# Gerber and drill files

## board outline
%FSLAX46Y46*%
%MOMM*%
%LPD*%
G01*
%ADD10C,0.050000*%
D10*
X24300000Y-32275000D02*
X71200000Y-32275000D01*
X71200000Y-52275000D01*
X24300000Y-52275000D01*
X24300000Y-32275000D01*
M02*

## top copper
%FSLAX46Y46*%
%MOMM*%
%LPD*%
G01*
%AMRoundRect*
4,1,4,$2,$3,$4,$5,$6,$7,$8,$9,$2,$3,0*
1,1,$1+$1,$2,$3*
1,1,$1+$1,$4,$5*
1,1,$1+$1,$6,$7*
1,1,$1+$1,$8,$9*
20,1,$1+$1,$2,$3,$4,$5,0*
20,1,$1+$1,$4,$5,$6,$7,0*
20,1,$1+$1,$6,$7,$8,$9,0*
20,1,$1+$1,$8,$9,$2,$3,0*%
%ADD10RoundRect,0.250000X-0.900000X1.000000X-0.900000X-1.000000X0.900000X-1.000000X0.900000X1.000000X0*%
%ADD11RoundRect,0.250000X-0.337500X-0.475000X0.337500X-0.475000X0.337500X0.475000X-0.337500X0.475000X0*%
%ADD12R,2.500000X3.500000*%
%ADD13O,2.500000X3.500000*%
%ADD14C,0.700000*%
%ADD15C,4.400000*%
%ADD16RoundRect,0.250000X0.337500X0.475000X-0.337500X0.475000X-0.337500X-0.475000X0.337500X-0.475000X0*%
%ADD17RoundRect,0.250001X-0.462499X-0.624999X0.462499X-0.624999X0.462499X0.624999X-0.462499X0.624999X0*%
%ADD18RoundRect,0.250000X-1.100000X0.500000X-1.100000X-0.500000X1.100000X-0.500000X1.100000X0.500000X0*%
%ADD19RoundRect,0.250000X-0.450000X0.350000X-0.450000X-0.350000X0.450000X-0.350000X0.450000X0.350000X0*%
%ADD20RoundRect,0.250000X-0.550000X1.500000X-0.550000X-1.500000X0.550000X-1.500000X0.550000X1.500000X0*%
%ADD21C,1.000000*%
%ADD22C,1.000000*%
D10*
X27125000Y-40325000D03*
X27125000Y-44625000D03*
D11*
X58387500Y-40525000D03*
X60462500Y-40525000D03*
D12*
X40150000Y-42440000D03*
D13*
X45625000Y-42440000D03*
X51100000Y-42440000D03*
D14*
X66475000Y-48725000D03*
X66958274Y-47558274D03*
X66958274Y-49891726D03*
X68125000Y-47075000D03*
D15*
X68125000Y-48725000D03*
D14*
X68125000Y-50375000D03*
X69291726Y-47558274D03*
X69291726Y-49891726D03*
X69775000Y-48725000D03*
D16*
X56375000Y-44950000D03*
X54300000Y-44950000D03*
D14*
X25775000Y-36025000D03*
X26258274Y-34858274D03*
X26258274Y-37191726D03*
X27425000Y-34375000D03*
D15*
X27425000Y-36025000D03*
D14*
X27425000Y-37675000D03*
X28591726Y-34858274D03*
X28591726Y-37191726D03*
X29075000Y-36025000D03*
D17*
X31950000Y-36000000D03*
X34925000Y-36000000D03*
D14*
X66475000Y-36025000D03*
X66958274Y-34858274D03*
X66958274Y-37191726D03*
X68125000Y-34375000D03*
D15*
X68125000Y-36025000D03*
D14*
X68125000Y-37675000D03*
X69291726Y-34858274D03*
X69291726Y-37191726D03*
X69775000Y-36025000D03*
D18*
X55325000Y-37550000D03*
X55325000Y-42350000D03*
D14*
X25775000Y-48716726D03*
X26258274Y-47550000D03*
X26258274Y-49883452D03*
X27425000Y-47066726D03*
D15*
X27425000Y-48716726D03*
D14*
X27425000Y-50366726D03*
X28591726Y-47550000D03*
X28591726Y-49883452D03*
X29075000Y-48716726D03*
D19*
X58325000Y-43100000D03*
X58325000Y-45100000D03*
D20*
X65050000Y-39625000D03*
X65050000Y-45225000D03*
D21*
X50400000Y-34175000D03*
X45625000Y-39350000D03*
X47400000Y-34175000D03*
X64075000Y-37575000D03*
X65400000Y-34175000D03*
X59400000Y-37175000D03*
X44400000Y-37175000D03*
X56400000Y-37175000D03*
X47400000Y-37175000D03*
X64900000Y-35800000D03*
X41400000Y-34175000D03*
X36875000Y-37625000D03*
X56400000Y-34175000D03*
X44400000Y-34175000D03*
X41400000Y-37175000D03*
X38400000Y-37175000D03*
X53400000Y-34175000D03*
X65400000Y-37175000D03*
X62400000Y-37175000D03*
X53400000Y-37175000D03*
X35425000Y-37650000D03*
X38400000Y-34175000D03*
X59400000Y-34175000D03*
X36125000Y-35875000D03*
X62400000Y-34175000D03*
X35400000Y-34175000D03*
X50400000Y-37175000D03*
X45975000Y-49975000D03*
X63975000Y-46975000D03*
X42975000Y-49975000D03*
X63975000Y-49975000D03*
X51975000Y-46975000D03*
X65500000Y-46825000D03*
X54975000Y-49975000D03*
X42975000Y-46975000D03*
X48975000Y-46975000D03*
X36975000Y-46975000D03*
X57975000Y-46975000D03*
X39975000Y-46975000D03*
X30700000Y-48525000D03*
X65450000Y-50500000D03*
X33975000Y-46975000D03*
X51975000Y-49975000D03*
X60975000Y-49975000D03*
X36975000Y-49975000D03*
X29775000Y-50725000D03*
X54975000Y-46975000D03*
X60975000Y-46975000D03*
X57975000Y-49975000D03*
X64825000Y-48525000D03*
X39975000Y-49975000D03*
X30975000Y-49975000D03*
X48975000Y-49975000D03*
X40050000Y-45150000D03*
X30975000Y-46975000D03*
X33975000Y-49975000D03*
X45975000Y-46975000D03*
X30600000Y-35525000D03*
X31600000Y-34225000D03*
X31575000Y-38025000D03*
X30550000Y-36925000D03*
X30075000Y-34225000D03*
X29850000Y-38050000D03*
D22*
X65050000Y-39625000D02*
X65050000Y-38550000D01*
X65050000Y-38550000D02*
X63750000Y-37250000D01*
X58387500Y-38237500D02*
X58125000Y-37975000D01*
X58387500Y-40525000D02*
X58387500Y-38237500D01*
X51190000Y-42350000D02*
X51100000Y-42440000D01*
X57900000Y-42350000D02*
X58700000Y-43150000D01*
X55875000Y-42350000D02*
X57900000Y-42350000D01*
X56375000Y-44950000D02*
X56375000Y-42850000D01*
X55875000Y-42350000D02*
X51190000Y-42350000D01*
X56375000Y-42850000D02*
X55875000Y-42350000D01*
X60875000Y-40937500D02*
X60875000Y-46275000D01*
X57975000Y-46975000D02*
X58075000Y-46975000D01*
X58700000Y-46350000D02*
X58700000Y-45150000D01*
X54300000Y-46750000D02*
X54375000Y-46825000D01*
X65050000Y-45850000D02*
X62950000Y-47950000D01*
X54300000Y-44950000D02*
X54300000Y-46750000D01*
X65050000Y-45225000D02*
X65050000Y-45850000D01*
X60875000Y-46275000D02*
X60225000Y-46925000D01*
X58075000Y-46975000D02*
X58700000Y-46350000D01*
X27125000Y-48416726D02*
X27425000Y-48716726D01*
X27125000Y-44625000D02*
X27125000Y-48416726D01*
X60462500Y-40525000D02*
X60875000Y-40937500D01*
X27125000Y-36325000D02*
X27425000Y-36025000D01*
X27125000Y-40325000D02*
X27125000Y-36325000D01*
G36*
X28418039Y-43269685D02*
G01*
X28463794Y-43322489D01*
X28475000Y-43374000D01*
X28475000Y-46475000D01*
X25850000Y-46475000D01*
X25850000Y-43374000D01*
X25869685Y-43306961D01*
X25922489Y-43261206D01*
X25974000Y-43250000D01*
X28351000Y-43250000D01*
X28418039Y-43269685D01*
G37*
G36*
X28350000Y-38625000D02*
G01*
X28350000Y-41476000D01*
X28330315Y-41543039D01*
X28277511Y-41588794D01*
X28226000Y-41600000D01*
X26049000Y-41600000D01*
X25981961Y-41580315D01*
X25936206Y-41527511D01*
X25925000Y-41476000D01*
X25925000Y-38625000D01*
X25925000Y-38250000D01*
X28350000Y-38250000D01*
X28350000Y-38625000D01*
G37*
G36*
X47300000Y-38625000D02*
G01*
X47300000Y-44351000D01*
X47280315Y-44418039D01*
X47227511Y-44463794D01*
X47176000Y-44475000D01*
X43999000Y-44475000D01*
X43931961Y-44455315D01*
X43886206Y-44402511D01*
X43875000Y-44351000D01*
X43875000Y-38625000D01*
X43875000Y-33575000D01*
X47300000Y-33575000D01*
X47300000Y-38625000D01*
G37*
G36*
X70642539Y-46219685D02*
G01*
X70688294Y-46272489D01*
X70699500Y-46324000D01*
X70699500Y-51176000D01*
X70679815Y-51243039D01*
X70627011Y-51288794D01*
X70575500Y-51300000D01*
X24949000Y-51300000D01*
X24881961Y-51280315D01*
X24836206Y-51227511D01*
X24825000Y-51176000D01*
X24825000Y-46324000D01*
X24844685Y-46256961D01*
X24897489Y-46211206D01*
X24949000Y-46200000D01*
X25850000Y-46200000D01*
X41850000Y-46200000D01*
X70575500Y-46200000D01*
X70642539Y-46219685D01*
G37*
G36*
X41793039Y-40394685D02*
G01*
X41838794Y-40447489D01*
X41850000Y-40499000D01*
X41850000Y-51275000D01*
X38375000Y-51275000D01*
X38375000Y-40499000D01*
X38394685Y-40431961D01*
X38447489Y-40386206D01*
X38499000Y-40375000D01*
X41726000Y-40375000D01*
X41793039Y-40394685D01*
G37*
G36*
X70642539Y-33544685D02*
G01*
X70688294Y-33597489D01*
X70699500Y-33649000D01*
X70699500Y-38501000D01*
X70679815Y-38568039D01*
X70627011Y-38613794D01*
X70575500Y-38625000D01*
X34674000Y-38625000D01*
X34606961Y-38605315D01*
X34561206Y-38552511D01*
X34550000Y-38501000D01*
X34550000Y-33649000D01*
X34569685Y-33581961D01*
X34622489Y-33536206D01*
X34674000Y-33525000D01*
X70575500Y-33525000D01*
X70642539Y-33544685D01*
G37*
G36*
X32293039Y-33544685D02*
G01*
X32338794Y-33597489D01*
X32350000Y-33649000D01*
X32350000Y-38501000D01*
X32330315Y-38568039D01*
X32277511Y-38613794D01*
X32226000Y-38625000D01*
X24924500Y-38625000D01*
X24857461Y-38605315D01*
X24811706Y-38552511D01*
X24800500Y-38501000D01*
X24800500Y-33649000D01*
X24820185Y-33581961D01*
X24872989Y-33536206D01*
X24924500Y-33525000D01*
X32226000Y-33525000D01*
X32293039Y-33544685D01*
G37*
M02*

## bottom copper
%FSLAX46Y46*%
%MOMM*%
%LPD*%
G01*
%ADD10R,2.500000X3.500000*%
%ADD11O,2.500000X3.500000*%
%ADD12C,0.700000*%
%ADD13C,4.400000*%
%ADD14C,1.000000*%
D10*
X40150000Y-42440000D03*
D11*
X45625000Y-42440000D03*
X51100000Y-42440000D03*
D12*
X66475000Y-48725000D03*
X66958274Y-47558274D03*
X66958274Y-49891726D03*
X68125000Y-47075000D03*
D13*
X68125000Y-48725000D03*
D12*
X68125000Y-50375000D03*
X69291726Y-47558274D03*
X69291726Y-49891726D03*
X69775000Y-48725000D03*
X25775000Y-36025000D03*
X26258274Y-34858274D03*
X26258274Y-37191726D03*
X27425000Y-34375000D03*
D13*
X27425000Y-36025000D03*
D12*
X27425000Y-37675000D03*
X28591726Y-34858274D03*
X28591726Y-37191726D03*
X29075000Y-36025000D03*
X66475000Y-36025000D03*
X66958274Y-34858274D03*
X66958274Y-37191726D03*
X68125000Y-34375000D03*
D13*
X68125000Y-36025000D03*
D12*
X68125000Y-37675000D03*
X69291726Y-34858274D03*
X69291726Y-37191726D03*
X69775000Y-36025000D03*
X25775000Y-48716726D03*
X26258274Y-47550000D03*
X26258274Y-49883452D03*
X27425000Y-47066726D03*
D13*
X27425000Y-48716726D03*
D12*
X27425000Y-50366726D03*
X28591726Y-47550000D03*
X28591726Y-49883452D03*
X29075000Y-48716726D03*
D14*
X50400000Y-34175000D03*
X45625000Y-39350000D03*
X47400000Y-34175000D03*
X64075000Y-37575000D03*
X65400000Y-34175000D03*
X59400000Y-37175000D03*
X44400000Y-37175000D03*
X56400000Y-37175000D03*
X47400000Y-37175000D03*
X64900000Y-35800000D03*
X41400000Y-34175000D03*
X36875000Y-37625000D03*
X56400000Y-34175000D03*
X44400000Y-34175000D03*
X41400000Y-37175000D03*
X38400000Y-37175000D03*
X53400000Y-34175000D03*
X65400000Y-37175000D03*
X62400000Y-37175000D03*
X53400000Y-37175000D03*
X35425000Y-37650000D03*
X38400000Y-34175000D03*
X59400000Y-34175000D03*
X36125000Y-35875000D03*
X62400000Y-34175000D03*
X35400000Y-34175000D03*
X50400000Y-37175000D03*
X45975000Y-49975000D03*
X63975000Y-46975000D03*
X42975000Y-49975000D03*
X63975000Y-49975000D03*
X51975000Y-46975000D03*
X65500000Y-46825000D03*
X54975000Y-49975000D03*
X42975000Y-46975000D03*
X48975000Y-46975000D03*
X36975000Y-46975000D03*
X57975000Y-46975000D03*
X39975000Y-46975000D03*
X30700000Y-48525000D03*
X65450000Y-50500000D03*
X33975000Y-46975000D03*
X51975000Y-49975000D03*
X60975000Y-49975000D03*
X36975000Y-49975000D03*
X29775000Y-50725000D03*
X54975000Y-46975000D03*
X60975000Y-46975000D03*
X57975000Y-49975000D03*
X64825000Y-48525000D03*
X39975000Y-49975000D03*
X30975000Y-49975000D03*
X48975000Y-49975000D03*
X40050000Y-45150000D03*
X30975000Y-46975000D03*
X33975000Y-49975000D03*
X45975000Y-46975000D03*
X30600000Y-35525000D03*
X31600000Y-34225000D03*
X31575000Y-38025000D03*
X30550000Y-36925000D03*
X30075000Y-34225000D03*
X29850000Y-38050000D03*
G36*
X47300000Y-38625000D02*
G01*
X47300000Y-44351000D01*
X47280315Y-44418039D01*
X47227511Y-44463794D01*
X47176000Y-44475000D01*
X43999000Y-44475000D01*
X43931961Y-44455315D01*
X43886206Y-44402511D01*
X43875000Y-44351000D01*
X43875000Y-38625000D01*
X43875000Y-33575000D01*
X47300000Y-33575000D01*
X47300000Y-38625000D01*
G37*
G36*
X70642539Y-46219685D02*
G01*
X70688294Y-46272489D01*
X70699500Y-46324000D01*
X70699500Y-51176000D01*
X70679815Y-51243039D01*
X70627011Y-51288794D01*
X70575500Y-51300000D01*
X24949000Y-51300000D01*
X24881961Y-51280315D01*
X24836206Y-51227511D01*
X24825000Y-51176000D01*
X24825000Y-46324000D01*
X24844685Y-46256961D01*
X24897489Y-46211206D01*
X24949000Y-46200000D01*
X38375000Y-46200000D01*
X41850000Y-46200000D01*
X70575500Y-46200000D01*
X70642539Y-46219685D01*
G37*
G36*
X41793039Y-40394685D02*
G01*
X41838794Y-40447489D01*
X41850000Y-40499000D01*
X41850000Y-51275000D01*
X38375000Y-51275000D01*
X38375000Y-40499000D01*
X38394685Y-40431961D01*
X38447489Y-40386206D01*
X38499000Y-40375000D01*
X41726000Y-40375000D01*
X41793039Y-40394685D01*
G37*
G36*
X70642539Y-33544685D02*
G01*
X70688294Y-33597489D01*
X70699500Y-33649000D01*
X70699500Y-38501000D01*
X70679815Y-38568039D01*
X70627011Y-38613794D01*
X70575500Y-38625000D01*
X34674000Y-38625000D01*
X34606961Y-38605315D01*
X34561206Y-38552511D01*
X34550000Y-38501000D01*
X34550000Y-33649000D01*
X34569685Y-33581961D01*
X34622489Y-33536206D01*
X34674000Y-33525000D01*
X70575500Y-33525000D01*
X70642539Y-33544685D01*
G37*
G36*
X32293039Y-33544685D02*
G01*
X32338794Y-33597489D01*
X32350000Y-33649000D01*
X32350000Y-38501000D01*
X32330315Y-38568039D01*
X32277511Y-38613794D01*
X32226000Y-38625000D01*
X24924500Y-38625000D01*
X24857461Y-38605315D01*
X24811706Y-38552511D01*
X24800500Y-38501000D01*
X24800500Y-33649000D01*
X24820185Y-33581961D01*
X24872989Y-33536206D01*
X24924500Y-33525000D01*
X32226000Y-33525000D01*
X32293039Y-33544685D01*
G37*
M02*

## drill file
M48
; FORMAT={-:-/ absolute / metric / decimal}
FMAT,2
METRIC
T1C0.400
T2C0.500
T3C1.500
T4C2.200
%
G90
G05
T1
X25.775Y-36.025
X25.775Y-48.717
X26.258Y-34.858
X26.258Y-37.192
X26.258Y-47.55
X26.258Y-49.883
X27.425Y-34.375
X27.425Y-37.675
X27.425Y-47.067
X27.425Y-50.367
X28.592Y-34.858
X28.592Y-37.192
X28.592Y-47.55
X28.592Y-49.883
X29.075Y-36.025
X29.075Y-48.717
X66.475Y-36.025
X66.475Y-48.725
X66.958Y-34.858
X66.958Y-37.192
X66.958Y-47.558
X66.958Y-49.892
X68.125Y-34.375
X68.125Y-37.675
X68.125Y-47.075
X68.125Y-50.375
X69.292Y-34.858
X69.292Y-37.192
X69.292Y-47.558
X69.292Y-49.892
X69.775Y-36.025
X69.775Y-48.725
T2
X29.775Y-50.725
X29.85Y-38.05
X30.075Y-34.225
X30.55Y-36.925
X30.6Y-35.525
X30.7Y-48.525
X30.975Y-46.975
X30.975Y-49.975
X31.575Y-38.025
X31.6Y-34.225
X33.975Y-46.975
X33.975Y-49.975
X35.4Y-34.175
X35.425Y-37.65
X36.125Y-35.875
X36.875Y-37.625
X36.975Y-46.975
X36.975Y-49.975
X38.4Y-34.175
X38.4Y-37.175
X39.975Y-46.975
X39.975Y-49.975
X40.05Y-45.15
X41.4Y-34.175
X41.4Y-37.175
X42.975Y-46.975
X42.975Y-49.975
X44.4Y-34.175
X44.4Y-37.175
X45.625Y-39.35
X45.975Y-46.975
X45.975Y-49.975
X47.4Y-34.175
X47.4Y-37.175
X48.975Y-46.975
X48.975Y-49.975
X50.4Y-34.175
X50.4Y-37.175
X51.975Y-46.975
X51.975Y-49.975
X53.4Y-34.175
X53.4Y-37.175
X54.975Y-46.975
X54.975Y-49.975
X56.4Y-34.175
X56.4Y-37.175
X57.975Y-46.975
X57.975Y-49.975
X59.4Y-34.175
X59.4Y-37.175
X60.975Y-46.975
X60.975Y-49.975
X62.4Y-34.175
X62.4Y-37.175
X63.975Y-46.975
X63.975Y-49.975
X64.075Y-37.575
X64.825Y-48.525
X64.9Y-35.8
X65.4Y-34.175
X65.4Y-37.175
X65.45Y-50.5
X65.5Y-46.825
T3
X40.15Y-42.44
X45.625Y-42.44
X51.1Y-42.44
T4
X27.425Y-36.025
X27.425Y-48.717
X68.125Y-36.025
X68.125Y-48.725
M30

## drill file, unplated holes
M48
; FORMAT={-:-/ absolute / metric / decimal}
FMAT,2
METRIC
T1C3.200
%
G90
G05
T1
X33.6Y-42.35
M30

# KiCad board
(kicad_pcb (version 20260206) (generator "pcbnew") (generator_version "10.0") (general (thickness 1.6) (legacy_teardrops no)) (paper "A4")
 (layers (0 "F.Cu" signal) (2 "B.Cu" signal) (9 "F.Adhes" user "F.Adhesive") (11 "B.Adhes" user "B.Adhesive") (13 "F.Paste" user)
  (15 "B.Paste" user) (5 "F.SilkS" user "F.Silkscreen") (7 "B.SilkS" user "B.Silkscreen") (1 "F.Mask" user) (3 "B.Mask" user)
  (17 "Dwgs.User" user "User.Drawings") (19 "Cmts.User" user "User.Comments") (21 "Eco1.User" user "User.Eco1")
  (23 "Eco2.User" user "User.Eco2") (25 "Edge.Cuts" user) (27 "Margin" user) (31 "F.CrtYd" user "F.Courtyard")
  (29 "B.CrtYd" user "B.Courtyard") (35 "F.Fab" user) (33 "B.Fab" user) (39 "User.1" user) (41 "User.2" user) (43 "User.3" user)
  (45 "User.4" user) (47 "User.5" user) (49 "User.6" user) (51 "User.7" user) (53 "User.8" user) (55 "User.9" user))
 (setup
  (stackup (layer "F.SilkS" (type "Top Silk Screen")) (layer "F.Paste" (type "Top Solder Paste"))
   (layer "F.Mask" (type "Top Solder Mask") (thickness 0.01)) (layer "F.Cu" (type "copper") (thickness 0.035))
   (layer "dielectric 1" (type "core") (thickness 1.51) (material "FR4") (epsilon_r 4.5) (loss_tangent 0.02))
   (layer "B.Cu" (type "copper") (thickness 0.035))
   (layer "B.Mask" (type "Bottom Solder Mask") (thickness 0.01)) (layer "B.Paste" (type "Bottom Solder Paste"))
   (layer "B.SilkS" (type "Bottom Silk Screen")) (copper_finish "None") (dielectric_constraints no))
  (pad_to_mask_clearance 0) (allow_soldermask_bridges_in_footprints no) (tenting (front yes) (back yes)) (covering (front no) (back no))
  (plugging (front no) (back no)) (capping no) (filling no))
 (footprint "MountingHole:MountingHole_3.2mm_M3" (layer "F.Cu") (at 33.6 42.35)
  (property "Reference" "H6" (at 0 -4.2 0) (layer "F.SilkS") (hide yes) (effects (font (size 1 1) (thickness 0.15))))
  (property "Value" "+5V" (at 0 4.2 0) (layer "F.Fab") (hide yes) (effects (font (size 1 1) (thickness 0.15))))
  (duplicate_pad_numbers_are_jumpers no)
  (pad "" np_thru_hole circle (at 0 0) (size 3.2 3.2) (drill 3.2) (layers "*.Cu" "*.Mask")))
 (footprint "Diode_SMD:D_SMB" (layer "F.Cu") (at 27.125 42.475 -90)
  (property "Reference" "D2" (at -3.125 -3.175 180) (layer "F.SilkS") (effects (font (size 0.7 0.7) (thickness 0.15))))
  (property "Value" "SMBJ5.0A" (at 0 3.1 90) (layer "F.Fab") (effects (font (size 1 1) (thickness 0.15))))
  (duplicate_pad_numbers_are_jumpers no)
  (pad "1" smd roundrect (at -2.15 0 270) (size 2.5 2.3) (layers "F.Cu" "F.Mask" "F.Paste") (roundrect_rratio 0.1086956522) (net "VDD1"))
  (pad "2" smd roundrect (at 2.15 0 270) (size 2.5 2.3) (layers "F.Cu" "F.Mask" "F.Paste") (roundrect_rratio 0.1086956522) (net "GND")))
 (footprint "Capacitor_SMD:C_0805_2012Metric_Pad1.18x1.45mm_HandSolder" (layer "F.Cu") (at 59.425 40.525)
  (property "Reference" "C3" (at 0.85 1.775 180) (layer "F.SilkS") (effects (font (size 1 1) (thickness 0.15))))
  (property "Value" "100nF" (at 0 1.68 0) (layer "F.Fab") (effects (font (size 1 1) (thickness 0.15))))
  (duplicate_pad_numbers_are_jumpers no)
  (pad "1" smd roundrect (at -1.0375 0) (size 1.175 1.45) (layers "F.Cu" "F.Mask" "F.Paste") (roundrect_rratio 0.212766) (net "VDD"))
  (pad "2" smd roundrect (at 1.0375 0) (size 1.175 1.45) (layers "F.Cu" "F.Mask" "F.Paste") (roundrect_rratio 0.212766) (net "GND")))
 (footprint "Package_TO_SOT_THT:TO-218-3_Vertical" (layer "F.Cu") (at 40.15 42.44)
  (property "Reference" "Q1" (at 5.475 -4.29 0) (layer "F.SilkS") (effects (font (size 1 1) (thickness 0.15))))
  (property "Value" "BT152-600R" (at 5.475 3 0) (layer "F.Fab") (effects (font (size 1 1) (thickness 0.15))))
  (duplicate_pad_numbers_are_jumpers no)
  (pad "1" thru_hole rect (at 0 0) (size 2.5 3.5) (drill 1.5) (layers "*.Cu" "*.Mask") (remove_unused_layers no) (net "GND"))
  (pad "2" thru_hole oval (at 5.475 0) (size 2.5 3.5) (drill 1.5) (layers "*.Cu" "*.Mask") (remove_unused_layers no) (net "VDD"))
  (pad "3" thru_hole oval (at 10.95 0) (size 2.5 3.5) (drill 1.5) (layers "*.Cu" "*.Mask") (remove_unused_layers no) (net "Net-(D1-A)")))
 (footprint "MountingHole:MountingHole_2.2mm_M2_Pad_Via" (layer "F.Cu") (at 68.125 48.725)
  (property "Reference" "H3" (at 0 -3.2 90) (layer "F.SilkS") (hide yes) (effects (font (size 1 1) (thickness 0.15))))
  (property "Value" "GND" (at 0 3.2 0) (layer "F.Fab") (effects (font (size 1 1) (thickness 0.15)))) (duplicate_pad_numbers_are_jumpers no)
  (pad "1" thru_hole circle (at -1.65 0) (size 0.7 0.7) (drill 0.4) (layers "*.Cu" "*.Mask") (remove_unused_layers no) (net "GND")
   (zone_connect 2))
  (pad "1" thru_hole circle (at -1.166726 -1.166726) (size 0.7 0.7) (drill 0.4) (layers "*.Cu" "*.Mask") (remove_unused_layers no)
   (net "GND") (zone_connect 2))
  (pad "1" thru_hole circle (at -1.166726 1.166726) (size 0.7 0.7) (drill 0.4) (layers "*.Cu" "*.Mask") (remove_unused_layers no)
   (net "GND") (zone_connect 2))
  (pad "1" thru_hole circle (at 0 -1.65) (size 0.7 0.7) (drill 0.4) (layers "*.Cu" "*.Mask") (remove_unused_layers no) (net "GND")
   (zone_connect 2))
  (pad "1" thru_hole circle (at 0 0) (size 4.4 4.4) (drill 2.2) (layers "*.Cu" "*.Mask") (remove_unused_layers no) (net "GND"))
  (pad "1" thru_hole circle (at 0 1.65) (size 0.7 0.7) (drill 0.4) (layers "*.Cu" "*.Mask") (remove_unused_layers no) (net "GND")
   (zone_connect 2))
  (pad "1" thru_hole circle (at 1.166726 -1.166726) (size 0.7 0.7) (drill 0.4) (layers "*.Cu" "*.Mask") (remove_unused_layers no)
   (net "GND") (zone_connect 2))
  (pad "1" thru_hole circle (at 1.166726 1.166726) (size 0.7 0.7) (drill 0.4) (layers "*.Cu" "*.Mask") (remove_unused_layers no) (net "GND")
   (zone_connect 2))
  (pad "1" thru_hole circle (at 1.65 0) (size 0.7 0.7) (drill 0.4) (layers "*.Cu" "*.Mask") (remove_unused_layers no) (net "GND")
   (zone_connect 2)))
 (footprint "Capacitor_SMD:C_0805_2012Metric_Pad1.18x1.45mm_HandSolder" (layer "F.Cu") (at 55.3375 44.95 180)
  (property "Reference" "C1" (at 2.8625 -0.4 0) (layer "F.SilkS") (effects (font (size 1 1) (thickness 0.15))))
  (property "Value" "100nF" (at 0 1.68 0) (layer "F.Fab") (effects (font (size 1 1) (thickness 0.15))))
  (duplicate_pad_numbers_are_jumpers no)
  (pad "1" smd roundrect (at -1.0375 0 180) (size 1.175 1.45) (layers "F.Cu" "F.Mask" "F.Paste") (roundrect_rratio 0.212766)
   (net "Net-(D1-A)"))
  (pad "2" smd roundrect (at 1.0375 0 180) (size 1.175 1.45) (layers "F.Cu" "F.Mask" "F.Paste") (roundrect_rratio 0.212766) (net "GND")))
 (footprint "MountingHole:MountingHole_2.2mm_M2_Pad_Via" (layer "F.Cu") (at 27.425 36.025)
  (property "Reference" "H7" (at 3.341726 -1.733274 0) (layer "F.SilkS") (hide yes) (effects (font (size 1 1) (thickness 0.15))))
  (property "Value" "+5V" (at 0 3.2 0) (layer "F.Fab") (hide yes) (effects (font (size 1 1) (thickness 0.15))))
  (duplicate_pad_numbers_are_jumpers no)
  (pad "1" thru_hole circle (at -1.65 0) (size 0.7 0.7) (drill 0.4) (layers "*.Cu" "*.Mask") (remove_unused_layers no) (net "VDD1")
   (zone_connect 2))
  (pad "1" thru_hole circle (at -1.166726 -1.166726) (size 0.7 0.7) (drill 0.4) (layers "*.Cu" "*.Mask") (remove_unused_layers no)
   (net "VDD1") (zone_connect 2))
  (pad "1" thru_hole circle (at -1.166726 1.166726) (size 0.7 0.7) (drill 0.4) (layers "*.Cu" "*.Mask") (remove_unused_layers no)
   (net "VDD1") (zone_connect 2))
  (pad "1" thru_hole circle (at 0 -1.65) (size 0.7 0.7) (drill 0.4) (layers "*.Cu" "*.Mask") (remove_unused_layers no) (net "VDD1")
   (zone_connect 2))
  (pad "1" thru_hole circle (at 0 0) (size 4.4 4.4) (drill 2.2) (layers "*.Cu" "*.Mask") (remove_unused_layers no) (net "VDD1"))
  (pad "1" thru_hole circle (at 0 1.65) (size 0.7 0.7) (drill 0.4) (layers "*.Cu" "*.Mask") (remove_unused_layers no) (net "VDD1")
   (zone_connect 2))
  (pad "1" thru_hole circle (at 1.166726 -1.166726) (size 0.7 0.7) (drill 0.4) (layers "*.Cu" "*.Mask") (remove_unused_layers no)
   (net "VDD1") (zone_connect 2))
  (pad "1" thru_hole circle (at 1.166726 1.166726) (size 0.7 0.7) (drill 0.4) (layers "*.Cu" "*.Mask") (remove_unused_layers no)
   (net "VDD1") (zone_connect 2))
  (pad "1" thru_hole circle (at 1.65 0) (size 0.7 0.7) (drill 0.4) (layers "*.Cu" "*.Mask") (remove_unused_layers no) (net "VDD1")
   (zone_connect 2)))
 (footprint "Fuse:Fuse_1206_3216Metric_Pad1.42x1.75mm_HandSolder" (layer "F.Cu") (at 33.4375 36)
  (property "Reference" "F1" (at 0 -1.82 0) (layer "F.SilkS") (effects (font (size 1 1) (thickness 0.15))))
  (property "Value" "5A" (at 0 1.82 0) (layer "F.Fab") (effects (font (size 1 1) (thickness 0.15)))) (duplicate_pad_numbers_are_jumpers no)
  (pad "1" smd roundrect (at -1.4875 0) (size 1.425 1.75) (layers "F.Cu" "F.Mask" "F.Paste") (roundrect_rratio 0.175439) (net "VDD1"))
  (pad "2" smd roundrect (at 1.4875 0) (size 1.425 1.75) (layers "F.Cu" "F.Mask" "F.Paste") (roundrect_rratio 0.175439) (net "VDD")))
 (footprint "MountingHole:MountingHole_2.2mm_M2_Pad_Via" (layer "F.Cu") (at 68.125 36.025)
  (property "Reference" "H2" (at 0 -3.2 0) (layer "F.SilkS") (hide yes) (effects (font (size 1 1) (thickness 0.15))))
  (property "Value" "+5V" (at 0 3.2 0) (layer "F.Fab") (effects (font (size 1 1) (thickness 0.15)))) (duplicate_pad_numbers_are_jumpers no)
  (pad "1" thru_hole circle (at -1.65 0) (size 0.7 0.7) (drill 0.4) (layers "*.Cu" "*.Mask") (remove_unused_layers no) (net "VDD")
   (zone_connect 2))
  (pad "1" thru_hole circle (at -1.166726 -1.166726) (size 0.7 0.7) (drill 0.4) (layers "*.Cu" "*.Mask") (remove_unused_layers no)
   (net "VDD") (zone_connect 2))
  (pad "1" thru_hole circle (at -1.166726 1.166726) (size 0.7 0.7) (drill 0.4) (layers "*.Cu" "*.Mask") (remove_unused_layers no)
   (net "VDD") (zone_connect 2))
  (pad "1" thru_hole circle (at 0 -1.65) (size 0.7 0.7) (drill 0.4) (layers "*.Cu" "*.Mask") (remove_unused_layers no) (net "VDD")
   (zone_connect 2))
  (pad "1" thru_hole circle (at 0 0) (size 4.4 4.4) (drill 2.2) (layers "*.Cu" "*.Mask") (remove_unused_layers no) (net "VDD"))
  (pad "1" thru_hole circle (at 0 1.65) (size 0.7 0.7) (drill 0.4) (layers "*.Cu" "*.Mask") (remove_unused_layers no) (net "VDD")
   (zone_connect 2))
  (pad "1" thru_hole circle (at 1.166726 -1.166726) (size 0.7 0.7) (drill 0.4) (layers "*.Cu" "*.Mask") (remove_unused_layers no)
   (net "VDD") (zone_connect 2))
  (pad "1" thru_hole circle (at 1.166726 1.166726) (size 0.7 0.7) (drill 0.4) (layers "*.Cu" "*.Mask") (remove_unused_layers no) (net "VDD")
   (zone_connect 2))
  (pad "1" thru_hole circle (at 1.65 0) (size 0.7 0.7) (drill 0.4) (layers "*.Cu" "*.Mask") (remove_unused_layers no) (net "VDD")
   (zone_connect 2)))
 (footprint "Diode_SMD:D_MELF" (layer "F.Cu") (at 55.325 39.95 -90)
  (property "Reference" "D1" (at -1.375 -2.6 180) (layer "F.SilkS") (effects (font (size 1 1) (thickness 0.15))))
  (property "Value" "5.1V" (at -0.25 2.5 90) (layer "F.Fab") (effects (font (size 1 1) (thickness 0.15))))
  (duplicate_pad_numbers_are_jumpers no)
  (pad "1" smd roundrect (at -2.4 0 270) (size 1.5 2.7) (layers "F.Cu" "F.Mask" "F.Paste") (roundrect_rratio 0.1666666667) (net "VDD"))
  (pad "2" smd roundrect (at 2.4 0 270) (size 1.5 2.7) (layers "F.Cu" "F.Mask" "F.Paste") (roundrect_rratio 0.1666666667) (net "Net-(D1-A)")))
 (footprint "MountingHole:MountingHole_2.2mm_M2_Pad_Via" (layer "F.Cu") (at 27.425 48.716726)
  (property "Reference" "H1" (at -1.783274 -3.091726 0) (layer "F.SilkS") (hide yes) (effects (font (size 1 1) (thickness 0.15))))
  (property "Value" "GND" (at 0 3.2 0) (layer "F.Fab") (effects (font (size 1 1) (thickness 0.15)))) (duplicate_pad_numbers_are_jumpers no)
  (pad "1" thru_hole circle (at -1.65 0) (size 0.7 0.7) (drill 0.4) (layers "*.Cu" "*.Mask") (remove_unused_layers no) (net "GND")
   (zone_connect 2))
  (pad "1" thru_hole circle (at -1.166726 -1.166726) (size 0.7 0.7) (drill 0.4) (layers "*.Cu" "*.Mask") (remove_unused_layers no)
   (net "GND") (zone_connect 2))
  (pad "1" thru_hole circle (at -1.166726 1.166726) (size 0.7 0.7) (drill 0.4) (layers "*.Cu" "*.Mask") (remove_unused_layers no)
   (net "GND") (zone_connect 2))
  (pad "1" thru_hole circle (at 0 -1.65) (size 0.7 0.7) (drill 0.4) (layers "*.Cu" "*.Mask") (remove_unused_layers no) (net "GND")
   (zone_connect 2))
  (pad "1" thru_hole circle (at 0 0) (size 4.4 4.4) (drill 2.2) (layers "*.Cu" "*.Mask") (remove_unused_layers no) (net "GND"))
  (pad "1" thru_hole circle (at 0 1.65) (size 0.7 0.7) (drill 0.4) (layers "*.Cu" "*.Mask") (remove_unused_layers no) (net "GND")
   (zone_connect 2))
  (pad "1" thru_hole circle (at 1.166726 -1.166726) (size 0.7 0.7) (drill 0.4) (layers "*.Cu" "*.Mask") (remove_unused_layers no)
   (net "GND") (zone_connect 2))
  (pad "1" thru_hole circle (at 1.166726 1.166726) (size 0.7 0.7) (drill 0.4) (layers "*.Cu" "*.Mask") (remove_unused_layers no) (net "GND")
   (zone_connect 2))
  (pad "1" thru_hole circle (at 1.65 0) (size 0.7 0.7) (drill 0.4) (layers "*.Cu" "*.Mask") (remove_unused_layers no) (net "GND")
   (zone_connect 2)))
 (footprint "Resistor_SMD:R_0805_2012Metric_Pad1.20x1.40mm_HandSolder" (layer "F.Cu") (at 58.325 44.1 -90)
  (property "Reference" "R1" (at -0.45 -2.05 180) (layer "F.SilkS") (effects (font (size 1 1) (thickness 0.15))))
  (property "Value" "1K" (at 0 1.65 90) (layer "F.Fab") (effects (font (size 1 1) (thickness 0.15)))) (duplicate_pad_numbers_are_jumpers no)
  (pad "1" smd roundrect (at -1 0 270) (size 1.2 1.4) (layers "F.Cu" "F.Mask" "F.Paste") (roundrect_rratio 0.208333) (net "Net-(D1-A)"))
  (pad "2" smd roundrect (at 1 0 270) (size 1.2 1.4) (layers "F.Cu" "F.Mask" "F.Paste") (roundrect_rratio 0.208333) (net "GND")))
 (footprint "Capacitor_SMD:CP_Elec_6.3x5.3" (layer "F.Cu") (at 65.05 42.425 -90)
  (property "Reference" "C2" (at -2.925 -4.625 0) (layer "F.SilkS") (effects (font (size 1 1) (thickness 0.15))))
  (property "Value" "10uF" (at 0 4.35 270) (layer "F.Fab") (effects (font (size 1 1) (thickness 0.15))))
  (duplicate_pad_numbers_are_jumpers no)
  (pad "1" smd roundrect (at -2.8 0 270) (size 3.5 1.6) (layers "F.Cu" "F.Mask" "F.Paste") (roundrect_rratio 0.15625) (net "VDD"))
  (pad "2" smd roundrect (at 2.8 0 270) (size 3.5 1.6) (layers "F.Cu" "F.Mask" "F.Paste") (roundrect_rratio 0.15625) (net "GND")))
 (gr_rect (start 24.3 32.275) (end 71.2 52.275) (stroke (width 0.05) (type default)) (fill no) (layer "Edge.Cuts"))
 (segment (start 27.125 36.325) (end 27.425 36.025) (width 1) (layer "F.Cu") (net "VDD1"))
 (segment (start 27.125 40.325) (end 27.125 36.325) (width 1) (layer "F.Cu") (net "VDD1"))
 (via (at 30.6 35.525) (size 1) (drill 0.5) (layers "F.Cu" "B.Cu") (free yes) (capping no) (covering (front no) (back no))
  (plugging (front no) (back no)) (filling no) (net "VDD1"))
 (via (at 31.6 34.225) (size 1) (drill 0.5) (layers "F.Cu" "B.Cu") (free yes) (capping no) (covering (front no) (back no))
  (plugging (front no) (back no)) (filling no) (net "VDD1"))
 (via (at 31.575 38.025) (size 1) (drill 0.5) (layers "F.Cu" "B.Cu") (free yes) (capping no) (covering (front no) (back no))
  (plugging (front no) (back no)) (filling no) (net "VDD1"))
 (via (at 30.55 36.925) (size 1) (drill 0.5) (layers "F.Cu" "B.Cu") (free yes) (capping no) (covering (front no) (back no))
  (plugging (front no) (back no)) (filling no) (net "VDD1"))
 (via (at 30.075 34.225) (size 1) (drill 0.5) (layers "F.Cu" "B.Cu") (free yes) (capping no) (covering (front no) (back no))
  (plugging (front no) (back no)) (filling no) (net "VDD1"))
 (via (at 29.85 38.05) (size 1) (drill 0.5) (layers "F.Cu" "B.Cu") (free yes) (capping no) (covering (front no) (back no))
  (plugging (front no) (back no)) (filling no) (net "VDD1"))
 (segment (start 60.875 40.9375) (end 60.875 46.275) (width 1) (layer "F.Cu") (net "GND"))
 (segment (start 57.975 46.975) (end 58.075 46.975) (width 1) (layer "F.Cu") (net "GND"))
 (segment (start 58.7 46.35) (end 58.7 45.15) (width 1) (layer "F.Cu") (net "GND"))
 (segment (start 54.3 46.75) (end 54.375 46.825) (width 1) (layer "F.Cu") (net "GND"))
 (segment (start 65.05 45.85) (end 62.95 47.95) (width 1) (layer "F.Cu") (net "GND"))
 (segment (start 54.3 44.95) (end 54.3 46.75) (width 1) (layer "F.Cu") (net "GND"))
 (segment (start 65.05 45.225) (end 65.05 45.85) (width 1) (layer "F.Cu") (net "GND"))
 (segment (start 60.875 46.275) (end 60.225 46.925) (width 1) (layer "F.Cu") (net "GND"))
 (segment (start 58.075 46.975) (end 58.7 46.35) (width 1) (layer "F.Cu") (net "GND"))
 (segment (start 27.125 48.416726) (end 27.425 48.716726) (width 1) (layer "F.Cu") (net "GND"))
 (segment (start 27.125 44.625) (end 27.125 48.416726) (width 1) (layer "F.Cu") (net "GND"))
 (segment (start 60.4625 40.525) (end 60.875 40.9375) (width 1) (layer "F.Cu") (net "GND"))
 (via (at 45.975 49.975) (size 1) (drill 0.5) (layers "F.Cu" "B.Cu") (free yes) (capping no) (covering (front no) (back no))
  (plugging (front no) (back no)) (filling no) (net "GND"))
 (via (at 63.975 46.975) (size 1) (drill 0.5) (layers "F.Cu" "B.Cu") (free yes) (capping no) (covering (front no) (back no))
  (plugging (front no) (back no)) (filling no) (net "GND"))
 (via (at 42.975 49.975) (size 1) (drill 0.5) (layers "F.Cu" "B.Cu") (free yes) (capping no) (covering (front no) (back no))
  (plugging (front no) (back no)) (filling no) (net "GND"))
 (via (at 63.975 49.975) (size 1) (drill 0.5) (layers "F.Cu" "B.Cu") (free yes) (capping no) (covering (front no) (back no))
  (plugging (front no) (back no)) (filling no) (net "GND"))
 (via (at 51.975 46.975) (size 1) (drill 0.5) (layers "F.Cu" "B.Cu") (free yes) (capping no) (covering (front no) (back no))
  (plugging (front no) (back no)) (filling no) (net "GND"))
 (via (at 65.5 46.825) (size 1) (drill 0.5) (layers "F.Cu" "B.Cu") (free yes) (capping no) (covering (front no) (back no))
  (plugging (front no) (back no)) (filling no) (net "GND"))
 (via (at 54.975 49.975) (size 1) (drill 0.5) (layers "F.Cu" "B.Cu") (free yes) (capping no) (covering (front no) (back no))
  (plugging (front no) (back no)) (filling no) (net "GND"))
 (via (at 42.975 46.975) (size 1) (drill 0.5) (layers "F.Cu" "B.Cu") (free yes) (capping no) (covering (front no) (back no))
  (plugging (front no) (back no)) (filling no) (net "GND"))
 (via (at 48.975 46.975) (size 1) (drill 0.5) (layers "F.Cu" "B.Cu") (free yes) (capping no) (covering (front no) (back no))
  (plugging (front no) (back no)) (filling no) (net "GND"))
 (via (at 36.975 46.975) (size 1) (drill 0.5) (layers "F.Cu" "B.Cu") (free yes) (capping no) (covering (front no) (back no))
  (plugging (front no) (back no)) (filling no) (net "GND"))
 (via (at 57.975 46.975) (size 1) (drill 0.5) (layers "F.Cu" "B.Cu") (free yes) (capping no) (covering (front no) (back no))
  (plugging (front no) (back no)) (filling no) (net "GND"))
 (via (at 39.975 46.975) (size 1) (drill 0.5) (layers "F.Cu" "B.Cu") (free yes) (capping no) (covering (front no) (back no))
  (plugging (front no) (back no)) (filling no) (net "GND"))
 (via (at 30.7 48.525) (size 1) (drill 0.5) (layers "F.Cu" "B.Cu") (free yes) (capping no) (covering (front no) (back no))
  (plugging (front no) (back no)) (filling no) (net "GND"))
 (via (at 65.45 50.5) (size 1) (drill 0.5) (layers "F.Cu" "B.Cu") (free yes) (capping no) (covering (front no) (back no))
  (plugging (front no) (back no)) (filling no) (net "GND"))
 (via (at 33.975 46.975) (size 1) (drill 0.5) (layers "F.Cu" "B.Cu") (free yes) (capping no) (covering (front no) (back no))
  (plugging (front no) (back no)) (filling no) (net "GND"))
 (via (at 51.975 49.975) (size 1) (drill 0.5) (layers "F.Cu" "B.Cu") (free yes) (capping no) (covering (front no) (back no))
  (plugging (front no) (back no)) (filling no) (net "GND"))
 (via (at 60.975 49.975) (size 1) (drill 0.5) (layers "F.Cu" "B.Cu") (free yes) (capping no) (covering (front no) (back no))
  (plugging (front no) (back no)) (filling no) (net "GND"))
 (via (at 36.975 49.975) (size 1) (drill 0.5) (layers "F.Cu" "B.Cu") (free yes) (capping no) (covering (front no) (back no))
  (plugging (front no) (back no)) (filling no) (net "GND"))
 (via (at 29.775 50.725) (size 1) (drill 0.5) (layers "F.Cu" "B.Cu") (free yes) (capping no) (covering (front no) (back no))
  (plugging (front no) (back no)) (filling no) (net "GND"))
 (via (at 54.975 46.975) (size 1) (drill 0.5) (layers "F.Cu" "B.Cu") (free yes) (capping no) (covering (front no) (back no))
  (plugging (front no) (back no)) (filling no) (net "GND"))
 (via (at 60.975 46.975) (size 1) (drill 0.5) (layers "F.Cu" "B.Cu") (free yes) (capping no) (covering (front no) (back no))
  (plugging (front no) (back no)) (filling no) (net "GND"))
 (via (at 57.975 49.975) (size 1) (drill 0.5) (layers "F.Cu" "B.Cu") (free yes) (capping no) (covering (front no) (back no))
  (plugging (front no) (back no)) (filling no) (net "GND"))
 (via (at 64.825 48.525) (size 1) (drill 0.5) (layers "F.Cu" "B.Cu") (free yes) (capping no) (covering (front no) (back no))
  (plugging (front no) (back no)) (filling no) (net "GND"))
 (via (at 39.975 49.975) (size 1) (drill 0.5) (layers "F.Cu" "B.Cu") (free yes) (capping no) (covering (front no) (back no))
  (plugging (front no) (back no)) (filling no) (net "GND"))
 (via (at 30.975 49.975) (size 1) (drill 0.5) (layers "F.Cu" "B.Cu") (free yes) (capping no) (covering (front no) (back no))
  (plugging (front no) (back no)) (filling no) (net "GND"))
 (via (at 48.975 49.975) (size 1) (drill 0.5) (layers "F.Cu" "B.Cu") (free yes) (capping no) (covering (front no) (back no))
  (plugging (front no) (back no)) (filling no) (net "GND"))
 (via (at 40.05 45.15) (size 1) (drill 0.5) (layers "F.Cu" "B.Cu") (free yes) (capping no) (covering (front no) (back no))
  (plugging (front no) (back no)) (filling no) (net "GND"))
 (via (at 30.975 46.975) (size 1) (drill 0.5) (layers "F.Cu" "B.Cu") (free yes) (capping no) (covering (front no) (back no))
  (plugging (front no) (back no)) (filling no) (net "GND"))
 (via (at 33.975 49.975) (size 1) (drill 0.5) (layers "F.Cu" "B.Cu") (free yes) (capping no) (covering (front no) (back no))
  (plugging (front no) (back no)) (filling no) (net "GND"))
 (via (at 45.975 46.975) (size 1) (drill 0.5) (layers "F.Cu" "B.Cu") (free yes) (capping no) (covering (front no) (back no))
  (plugging (front no) (back no)) (filling no) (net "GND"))
 (segment (start 65.05 39.625) (end 65.05 38.55) (width 1) (layer "F.Cu") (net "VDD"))
 (segment (start 65.05 38.55) (end 63.75 37.25) (width 1) (layer "F.Cu") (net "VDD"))
 (segment (start 58.3875 38.2375) (end 58.125 37.975) (width 1) (layer "F.Cu") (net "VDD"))
 (segment (start 58.3875 40.525) (end 58.3875 38.2375) (width 1) (layer "F.Cu") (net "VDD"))
 (via (at 50.4 34.175) (size 1) (drill 0.5) (layers "F.Cu" "B.Cu") (free yes) (capping no) (covering (front no) (back no))
  (plugging (front no) (back no)) (filling no) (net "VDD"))
 (via (at 45.625 39.35) (size 1) (drill 0.5) (layers "F.Cu" "B.Cu") (free yes) (capping no) (covering (front no) (back no))
  (plugging (front no) (back no)) (filling no) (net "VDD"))
 (via (at 47.4 34.175) (size 1) (drill 0.5) (layers "F.Cu" "B.Cu") (free yes) (capping no) (covering (front no) (back no))
  (plugging (front no) (back no)) (filling no) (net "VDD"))
 (via (at 64.075 37.575) (size 1) (drill 0.5) (layers "F.Cu" "B.Cu") (free yes) (capping no) (covering (front no) (back no))
  (plugging (front no) (back no)) (filling no) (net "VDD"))
 (via (at 65.4 34.175) (size 1) (drill 0.5) (layers "F.Cu" "B.Cu") (free yes) (capping no) (covering (front no) (back no))
  (plugging (front no) (back no)) (filling no) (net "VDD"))
 (via (at 59.4 37.175) (size 1) (drill 0.5) (layers "F.Cu" "B.Cu") (free yes) (capping no) (covering (front no) (back no))
  (plugging (front no) (back no)) (filling no) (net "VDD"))
 (via (at 44.4 37.175) (size 1) (drill 0.5) (layers "F.Cu" "B.Cu") (free yes) (capping no) (covering (front no) (back no))
  (plugging (front no) (back no)) (filling no) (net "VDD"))
 (via (at 56.4 37.175) (size 1) (drill 0.5) (layers "F.Cu" "B.Cu") (free yes) (capping no) (covering (front no) (back no))
  (plugging (front no) (back no)) (filling no) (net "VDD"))
 (via (at 47.4 37.175) (size 1) (drill 0.5) (layers "F.Cu" "B.Cu") (free yes) (capping no) (covering (front no) (back no))
  (plugging (front no) (back no)) (filling no) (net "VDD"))
 (via (at 64.9 35.8) (size 1) (drill 0.5) (layers "F.Cu" "B.Cu") (free yes) (capping no) (covering (front no) (back no))
  (plugging (front no) (back no)) (filling no) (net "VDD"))
 (via (at 41.4 34.175) (size 1) (drill 0.5) (layers "F.Cu" "B.Cu") (free yes) (capping no) (covering (front no) (back no))
  (plugging (front no) (back no)) (filling no) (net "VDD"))
 (via (at 36.875 37.625) (size 1) (drill 0.5) (layers "F.Cu" "B.Cu") (free yes) (capping no) (covering (front no) (back no))
  (plugging (front no) (back no)) (filling no) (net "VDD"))
 (via (at 56.4 34.175) (size 1) (drill 0.5) (layers "F.Cu" "B.Cu") (free yes) (capping no) (covering (front no) (back no))
  (plugging (front no) (back no)) (filling no) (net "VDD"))
 (via (at 44.4 34.175) (size 1) (drill 0.5) (layers "F.Cu" "B.Cu") (free yes) (capping no) (covering (front no) (back no))
  (plugging (front no) (back no)) (filling no) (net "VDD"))
 (via (at 41.4 37.175) (size 1) (drill 0.5) (layers "F.Cu" "B.Cu") (free yes) (capping no) (covering (front no) (back no))
  (plugging (front no) (back no)) (filling no) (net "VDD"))
 (via (at 38.4 37.175) (size 1) (drill 0.5) (layers "F.Cu" "B.Cu") (free yes) (capping no) (covering (front no) (back no))
  (plugging (front no) (back no)) (filling no) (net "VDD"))
 (via (at 53.4 34.175) (size 1) (drill 0.5) (layers "F.Cu" "B.Cu") (free yes) (capping no) (covering (front no) (back no))
  (plugging (front no) (back no)) (filling no) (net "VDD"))
 (via (at 65.4 37.175) (size 1) (drill 0.5) (layers "F.Cu" "B.Cu") (free yes) (capping no) (covering (front no) (back no))
  (plugging (front no) (back no)) (filling no) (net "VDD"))
 (via (at 62.4 37.175) (size 1) (drill 0.5) (layers "F.Cu" "B.Cu") (free yes) (capping no) (covering (front no) (back no))
  (plugging (front no) (back no)) (filling no) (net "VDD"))
 (via (at 53.4 37.175) (size 1) (drill 0.5) (layers "F.Cu" "B.Cu") (free yes) (capping no) (covering (front no) (back no))
  (plugging (front no) (back no)) (filling no) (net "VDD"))
 (via (at 35.425 37.65) (size 1) (drill 0.5) (layers "F.Cu" "B.Cu") (free yes) (capping no) (covering (front no) (back no))
  (plugging (front no) (back no)) (filling no) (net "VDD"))
 (via (at 38.4 34.175) (size 1) (drill 0.5) (layers "F.Cu" "B.Cu") (free yes) (capping no) (covering (front no) (back no))
  (plugging (front no) (back no)) (filling no) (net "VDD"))
 (via (at 59.4 34.175) (size 1) (drill 0.5) (layers "F.Cu" "B.Cu") (free yes) (capping no) (covering (front no) (back no))
  (plugging (front no) (back no)) (filling no) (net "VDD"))
 (via (at 36.125 35.875) (size 1) (drill 0.5) (layers "F.Cu" "B.Cu") (free yes) (capping no) (covering (front no) (back no))
  (plugging (front no) (back no)) (filling no) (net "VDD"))
 (via (at 62.4 34.175) (size 1) (drill 0.5) (layers "F.Cu" "B.Cu") (free yes) (capping no) (covering (front no) (back no))
  (plugging (front no) (back no)) (filling no) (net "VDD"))
 (via (at 35.4 34.175) (size 1) (drill 0.5) (layers "F.Cu" "B.Cu") (free yes) (capping no) (covering (front no) (back no))
  (plugging (front no) (back no)) (filling no) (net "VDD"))
 (via (at 50.4 37.175) (size 1) (drill 0.5) (layers "F.Cu" "B.Cu") (free yes) (capping no) (covering (front no) (back no))
  (plugging (front no) (back no)) (filling no) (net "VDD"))
 (segment (start 51.19 42.35) (end 51.1 42.44) (width 1) (layer "F.Cu") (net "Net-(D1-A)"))
 (segment (start 57.9 42.35) (end 58.7 43.15) (width 1) (layer "F.Cu") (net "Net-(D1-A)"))
 (segment (start 55.875 42.35) (end 57.9 42.35) (width 1) (layer "F.Cu") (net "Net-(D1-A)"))
 (segment (start 56.375 44.95) (end 56.375 42.85) (width 1) (layer "F.Cu") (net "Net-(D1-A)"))
 (segment (start 55.875 42.35) (end 51.19 42.35) (width 1) (layer "F.Cu") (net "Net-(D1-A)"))
 (segment (start 56.375 42.85) (end 55.875 42.35) (width 1) (layer "F.Cu") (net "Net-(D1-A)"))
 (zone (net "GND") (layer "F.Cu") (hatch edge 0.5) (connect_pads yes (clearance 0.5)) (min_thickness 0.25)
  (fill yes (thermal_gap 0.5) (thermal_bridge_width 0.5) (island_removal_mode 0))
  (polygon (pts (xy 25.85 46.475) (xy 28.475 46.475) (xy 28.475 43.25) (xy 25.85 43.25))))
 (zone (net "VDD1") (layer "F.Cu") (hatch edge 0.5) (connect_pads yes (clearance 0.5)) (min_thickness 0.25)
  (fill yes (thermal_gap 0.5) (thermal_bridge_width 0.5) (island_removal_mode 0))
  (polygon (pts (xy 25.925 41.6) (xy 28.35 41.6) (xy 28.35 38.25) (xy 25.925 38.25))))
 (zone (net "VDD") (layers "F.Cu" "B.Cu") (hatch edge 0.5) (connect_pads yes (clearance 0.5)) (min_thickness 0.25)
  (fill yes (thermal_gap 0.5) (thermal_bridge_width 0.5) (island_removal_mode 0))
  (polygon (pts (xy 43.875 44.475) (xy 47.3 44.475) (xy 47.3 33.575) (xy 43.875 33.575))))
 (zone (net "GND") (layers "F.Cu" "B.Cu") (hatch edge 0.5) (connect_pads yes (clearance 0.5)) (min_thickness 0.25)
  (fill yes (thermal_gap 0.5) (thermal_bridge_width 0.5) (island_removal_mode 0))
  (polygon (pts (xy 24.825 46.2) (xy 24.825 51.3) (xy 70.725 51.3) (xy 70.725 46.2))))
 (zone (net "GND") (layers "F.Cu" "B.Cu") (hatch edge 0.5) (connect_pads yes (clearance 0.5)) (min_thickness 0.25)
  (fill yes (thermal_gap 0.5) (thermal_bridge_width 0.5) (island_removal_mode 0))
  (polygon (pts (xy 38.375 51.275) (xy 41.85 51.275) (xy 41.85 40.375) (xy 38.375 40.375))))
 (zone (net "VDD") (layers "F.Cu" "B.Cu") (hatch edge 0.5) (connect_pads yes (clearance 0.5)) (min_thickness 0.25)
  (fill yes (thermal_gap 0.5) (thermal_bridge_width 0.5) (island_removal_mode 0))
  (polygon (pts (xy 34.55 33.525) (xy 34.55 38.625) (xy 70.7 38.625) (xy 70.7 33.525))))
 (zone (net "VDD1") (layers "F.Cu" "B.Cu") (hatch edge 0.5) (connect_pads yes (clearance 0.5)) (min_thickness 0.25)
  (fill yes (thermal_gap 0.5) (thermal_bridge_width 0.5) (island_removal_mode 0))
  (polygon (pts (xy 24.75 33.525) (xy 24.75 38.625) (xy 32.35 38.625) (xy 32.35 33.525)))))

